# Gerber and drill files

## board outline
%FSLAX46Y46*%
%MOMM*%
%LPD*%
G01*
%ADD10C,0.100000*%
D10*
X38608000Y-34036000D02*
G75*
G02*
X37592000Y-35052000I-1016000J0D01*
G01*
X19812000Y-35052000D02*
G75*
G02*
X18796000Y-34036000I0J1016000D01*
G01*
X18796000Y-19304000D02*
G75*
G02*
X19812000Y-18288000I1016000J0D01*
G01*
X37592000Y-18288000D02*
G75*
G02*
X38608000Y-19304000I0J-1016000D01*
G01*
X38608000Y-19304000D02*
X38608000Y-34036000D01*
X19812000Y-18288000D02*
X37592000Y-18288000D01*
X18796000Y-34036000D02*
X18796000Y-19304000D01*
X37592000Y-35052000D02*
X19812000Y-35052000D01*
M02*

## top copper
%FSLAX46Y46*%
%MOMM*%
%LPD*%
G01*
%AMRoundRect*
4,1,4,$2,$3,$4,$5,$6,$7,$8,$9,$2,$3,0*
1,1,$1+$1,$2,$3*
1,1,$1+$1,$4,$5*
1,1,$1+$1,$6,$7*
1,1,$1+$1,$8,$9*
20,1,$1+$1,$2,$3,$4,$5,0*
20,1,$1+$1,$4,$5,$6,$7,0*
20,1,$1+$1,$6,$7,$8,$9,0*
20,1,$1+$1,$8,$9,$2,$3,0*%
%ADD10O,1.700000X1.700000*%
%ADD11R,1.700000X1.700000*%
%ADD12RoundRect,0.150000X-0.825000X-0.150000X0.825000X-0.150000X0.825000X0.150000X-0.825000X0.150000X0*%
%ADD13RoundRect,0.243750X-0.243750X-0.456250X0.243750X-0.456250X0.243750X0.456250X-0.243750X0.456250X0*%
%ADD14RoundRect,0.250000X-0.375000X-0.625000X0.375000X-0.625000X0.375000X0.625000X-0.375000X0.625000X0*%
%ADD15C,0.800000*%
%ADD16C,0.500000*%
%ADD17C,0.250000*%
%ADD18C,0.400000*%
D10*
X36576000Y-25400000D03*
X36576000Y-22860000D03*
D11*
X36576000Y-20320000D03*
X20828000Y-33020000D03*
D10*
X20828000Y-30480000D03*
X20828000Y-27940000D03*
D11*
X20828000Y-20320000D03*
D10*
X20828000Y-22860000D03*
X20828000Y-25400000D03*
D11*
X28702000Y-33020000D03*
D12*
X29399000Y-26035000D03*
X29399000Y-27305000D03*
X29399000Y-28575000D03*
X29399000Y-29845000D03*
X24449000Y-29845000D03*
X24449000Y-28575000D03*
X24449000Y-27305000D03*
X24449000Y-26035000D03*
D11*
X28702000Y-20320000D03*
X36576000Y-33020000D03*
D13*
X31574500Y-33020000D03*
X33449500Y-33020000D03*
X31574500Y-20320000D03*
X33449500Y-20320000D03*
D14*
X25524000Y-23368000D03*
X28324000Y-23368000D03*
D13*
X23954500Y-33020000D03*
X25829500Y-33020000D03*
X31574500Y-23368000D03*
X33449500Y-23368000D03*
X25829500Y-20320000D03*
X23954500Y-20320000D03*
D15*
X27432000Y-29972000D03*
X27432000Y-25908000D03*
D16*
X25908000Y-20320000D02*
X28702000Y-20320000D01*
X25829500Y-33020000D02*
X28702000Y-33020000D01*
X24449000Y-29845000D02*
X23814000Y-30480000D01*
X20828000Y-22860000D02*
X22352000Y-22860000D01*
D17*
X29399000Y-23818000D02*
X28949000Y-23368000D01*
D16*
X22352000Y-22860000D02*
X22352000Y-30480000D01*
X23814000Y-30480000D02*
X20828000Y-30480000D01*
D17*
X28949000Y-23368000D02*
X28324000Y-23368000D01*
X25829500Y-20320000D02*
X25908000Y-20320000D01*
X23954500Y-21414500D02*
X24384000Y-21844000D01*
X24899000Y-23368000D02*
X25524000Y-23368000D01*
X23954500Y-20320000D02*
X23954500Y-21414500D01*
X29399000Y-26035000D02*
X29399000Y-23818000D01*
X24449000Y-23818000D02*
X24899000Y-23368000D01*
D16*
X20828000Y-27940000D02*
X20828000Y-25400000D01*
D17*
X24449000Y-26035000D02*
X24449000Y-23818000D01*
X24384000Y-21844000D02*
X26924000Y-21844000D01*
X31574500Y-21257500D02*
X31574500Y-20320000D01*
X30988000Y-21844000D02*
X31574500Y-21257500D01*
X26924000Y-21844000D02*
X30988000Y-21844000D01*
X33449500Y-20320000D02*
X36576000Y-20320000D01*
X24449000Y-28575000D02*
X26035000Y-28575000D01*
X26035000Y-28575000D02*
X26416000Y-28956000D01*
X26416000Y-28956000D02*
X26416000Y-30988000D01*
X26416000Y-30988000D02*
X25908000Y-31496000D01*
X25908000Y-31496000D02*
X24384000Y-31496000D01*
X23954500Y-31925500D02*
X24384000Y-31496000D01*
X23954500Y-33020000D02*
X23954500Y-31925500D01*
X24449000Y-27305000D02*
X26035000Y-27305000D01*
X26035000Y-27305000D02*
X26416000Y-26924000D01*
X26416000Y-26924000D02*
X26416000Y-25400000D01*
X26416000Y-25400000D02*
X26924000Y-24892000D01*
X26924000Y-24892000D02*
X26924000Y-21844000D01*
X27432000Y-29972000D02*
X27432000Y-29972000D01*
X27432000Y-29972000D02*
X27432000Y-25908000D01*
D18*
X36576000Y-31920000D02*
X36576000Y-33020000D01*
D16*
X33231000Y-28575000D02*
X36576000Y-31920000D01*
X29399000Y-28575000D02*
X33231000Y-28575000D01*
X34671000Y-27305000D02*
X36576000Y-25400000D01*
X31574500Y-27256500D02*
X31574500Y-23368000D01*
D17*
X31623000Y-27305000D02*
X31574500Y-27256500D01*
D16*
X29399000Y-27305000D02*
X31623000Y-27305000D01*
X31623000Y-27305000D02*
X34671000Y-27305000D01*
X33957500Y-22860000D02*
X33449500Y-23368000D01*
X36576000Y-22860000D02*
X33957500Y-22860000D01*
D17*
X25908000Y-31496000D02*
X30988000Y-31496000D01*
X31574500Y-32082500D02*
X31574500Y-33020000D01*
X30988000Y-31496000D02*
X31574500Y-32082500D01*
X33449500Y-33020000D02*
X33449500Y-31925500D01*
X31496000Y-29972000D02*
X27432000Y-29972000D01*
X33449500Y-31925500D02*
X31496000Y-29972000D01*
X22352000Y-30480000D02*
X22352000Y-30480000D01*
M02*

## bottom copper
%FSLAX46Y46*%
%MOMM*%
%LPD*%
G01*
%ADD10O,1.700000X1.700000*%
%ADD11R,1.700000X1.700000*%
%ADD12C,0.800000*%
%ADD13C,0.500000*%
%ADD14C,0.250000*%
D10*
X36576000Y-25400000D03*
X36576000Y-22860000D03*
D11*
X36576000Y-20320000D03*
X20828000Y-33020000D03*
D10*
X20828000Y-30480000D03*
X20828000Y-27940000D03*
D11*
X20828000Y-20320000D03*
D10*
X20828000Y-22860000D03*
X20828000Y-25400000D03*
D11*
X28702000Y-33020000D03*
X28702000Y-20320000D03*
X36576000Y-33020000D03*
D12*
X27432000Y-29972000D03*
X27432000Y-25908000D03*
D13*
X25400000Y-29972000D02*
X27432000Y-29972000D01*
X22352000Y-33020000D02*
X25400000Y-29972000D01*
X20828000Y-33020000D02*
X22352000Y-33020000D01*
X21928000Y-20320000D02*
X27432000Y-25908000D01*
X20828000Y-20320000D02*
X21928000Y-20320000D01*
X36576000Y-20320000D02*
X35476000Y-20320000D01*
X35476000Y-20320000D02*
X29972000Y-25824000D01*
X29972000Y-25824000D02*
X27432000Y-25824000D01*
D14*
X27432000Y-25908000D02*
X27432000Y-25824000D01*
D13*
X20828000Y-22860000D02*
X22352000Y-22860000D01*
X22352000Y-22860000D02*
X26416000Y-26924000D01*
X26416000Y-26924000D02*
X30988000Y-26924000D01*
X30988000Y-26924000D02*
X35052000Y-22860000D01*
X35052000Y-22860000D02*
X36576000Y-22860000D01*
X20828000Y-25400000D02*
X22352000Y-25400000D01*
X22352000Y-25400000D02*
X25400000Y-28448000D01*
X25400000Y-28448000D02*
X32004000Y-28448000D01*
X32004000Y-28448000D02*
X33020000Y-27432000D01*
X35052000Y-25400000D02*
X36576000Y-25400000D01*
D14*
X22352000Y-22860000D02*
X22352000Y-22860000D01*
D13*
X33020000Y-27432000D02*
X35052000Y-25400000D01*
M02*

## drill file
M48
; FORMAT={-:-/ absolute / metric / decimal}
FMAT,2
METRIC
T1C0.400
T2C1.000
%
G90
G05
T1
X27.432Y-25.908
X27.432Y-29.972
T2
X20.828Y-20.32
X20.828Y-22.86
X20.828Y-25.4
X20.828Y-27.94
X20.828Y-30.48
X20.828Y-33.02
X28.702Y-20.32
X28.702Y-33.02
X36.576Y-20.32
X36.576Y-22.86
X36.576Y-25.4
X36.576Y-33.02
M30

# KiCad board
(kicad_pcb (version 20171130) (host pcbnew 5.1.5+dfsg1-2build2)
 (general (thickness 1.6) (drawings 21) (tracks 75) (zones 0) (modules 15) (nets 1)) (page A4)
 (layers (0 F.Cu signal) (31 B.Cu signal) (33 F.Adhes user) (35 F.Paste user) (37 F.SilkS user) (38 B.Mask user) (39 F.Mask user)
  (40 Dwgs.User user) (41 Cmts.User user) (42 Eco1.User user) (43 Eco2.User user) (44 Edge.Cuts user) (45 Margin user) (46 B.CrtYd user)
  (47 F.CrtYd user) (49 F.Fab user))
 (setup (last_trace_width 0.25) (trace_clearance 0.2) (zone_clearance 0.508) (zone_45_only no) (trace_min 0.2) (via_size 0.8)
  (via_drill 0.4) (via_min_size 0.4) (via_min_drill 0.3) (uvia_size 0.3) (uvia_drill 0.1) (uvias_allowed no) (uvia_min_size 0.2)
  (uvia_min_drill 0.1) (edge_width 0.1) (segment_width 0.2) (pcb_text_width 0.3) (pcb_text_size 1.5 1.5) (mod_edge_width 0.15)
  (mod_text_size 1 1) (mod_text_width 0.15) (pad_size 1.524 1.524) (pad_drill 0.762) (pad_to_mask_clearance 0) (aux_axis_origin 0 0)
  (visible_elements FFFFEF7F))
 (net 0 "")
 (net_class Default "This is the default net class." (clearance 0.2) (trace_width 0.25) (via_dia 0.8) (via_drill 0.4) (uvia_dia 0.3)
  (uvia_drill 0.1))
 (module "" (layer F.Cu) (at 26.67 28.448)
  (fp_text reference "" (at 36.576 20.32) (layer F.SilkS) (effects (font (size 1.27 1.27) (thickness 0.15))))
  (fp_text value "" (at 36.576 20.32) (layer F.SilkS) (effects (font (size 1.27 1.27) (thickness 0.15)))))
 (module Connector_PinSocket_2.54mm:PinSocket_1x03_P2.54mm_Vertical (layer F.Cu) (at 36.576 20.32)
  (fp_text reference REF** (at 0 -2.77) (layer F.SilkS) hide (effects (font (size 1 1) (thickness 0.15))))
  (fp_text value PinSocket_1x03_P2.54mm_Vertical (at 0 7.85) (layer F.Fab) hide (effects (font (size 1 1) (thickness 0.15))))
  (pad 3 thru_hole oval (at 0 5.08) (size 1.7 1.7) (drill 1) (layers *.Cu *.Mask))
  (pad 2 thru_hole oval (at 0 2.54) (size 1.7 1.7) (drill 1) (layers *.Cu *.Mask))
  (pad 1 thru_hole rect (at 0 0) (size 1.7 1.7) (drill 1) (layers *.Cu *.Mask)))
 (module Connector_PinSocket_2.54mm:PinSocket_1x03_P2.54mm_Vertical (layer F.Cu) (at 20.828 33.02 180)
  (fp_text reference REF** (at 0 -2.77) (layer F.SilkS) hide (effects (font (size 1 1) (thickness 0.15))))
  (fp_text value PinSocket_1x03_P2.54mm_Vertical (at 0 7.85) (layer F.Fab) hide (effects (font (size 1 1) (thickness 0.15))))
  (pad 1 thru_hole rect (at 0 0 180) (size 1.7 1.7) (drill 1) (layers *.Cu *.Mask))
  (pad 2 thru_hole oval (at 0 2.54 180) (size 1.7 1.7) (drill 1) (layers *.Cu *.Mask))
  (pad 3 thru_hole oval (at 0 5.08 180) (size 1.7 1.7) (drill 1) (layers *.Cu *.Mask)))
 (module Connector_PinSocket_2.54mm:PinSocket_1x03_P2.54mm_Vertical (layer F.Cu) (at 20.828 20.32)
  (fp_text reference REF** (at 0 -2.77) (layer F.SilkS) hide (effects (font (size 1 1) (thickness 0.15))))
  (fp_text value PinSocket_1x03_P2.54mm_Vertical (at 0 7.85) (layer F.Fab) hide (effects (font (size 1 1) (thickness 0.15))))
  (pad 1 thru_hole rect (at 0 0) (size 1.7 1.7) (drill 1) (layers *.Cu *.Mask))
  (pad 2 thru_hole oval (at 0 2.54) (size 1.7 1.7) (drill 1) (layers *.Cu *.Mask))
  (pad 3 thru_hole oval (at 0 5.08) (size 1.7 1.7) (drill 1) (layers *.Cu *.Mask)))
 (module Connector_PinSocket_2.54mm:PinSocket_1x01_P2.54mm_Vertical (layer F.Cu) (at 28.702 33.02)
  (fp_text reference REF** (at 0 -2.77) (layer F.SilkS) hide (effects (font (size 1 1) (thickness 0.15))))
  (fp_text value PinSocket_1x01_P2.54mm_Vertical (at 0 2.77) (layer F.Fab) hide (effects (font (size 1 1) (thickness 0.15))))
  (pad 1 thru_hole rect (at 0 0) (size 1.7 1.7) (drill 1) (layers *.Cu *.Mask)))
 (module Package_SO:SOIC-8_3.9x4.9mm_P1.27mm (layer F.Cu) (at 26.924 27.94)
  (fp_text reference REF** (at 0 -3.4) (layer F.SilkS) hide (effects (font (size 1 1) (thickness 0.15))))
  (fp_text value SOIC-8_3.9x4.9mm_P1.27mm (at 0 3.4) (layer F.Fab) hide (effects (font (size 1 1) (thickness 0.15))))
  (pad 8 smd roundrect (at 2.475 -1.905) (size 1.95 0.6) (layers F.Cu F.Paste F.Mask) (roundrect_rratio 0.25))
  (pad 7 smd roundrect (at 2.475 -0.635) (size 1.95 0.6) (layers F.Cu F.Paste F.Mask) (roundrect_rratio 0.25))
  (pad 6 smd roundrect (at 2.475 0.635) (size 1.95 0.6) (layers F.Cu F.Paste F.Mask) (roundrect_rratio 0.25))
  (pad 5 smd roundrect (at 2.475 1.905) (size 1.95 0.6) (layers F.Cu F.Paste F.Mask) (roundrect_rratio 0.25))
  (pad 4 smd roundrect (at -2.475 1.905) (size 1.95 0.6) (layers F.Cu F.Paste F.Mask) (roundrect_rratio 0.25))
  (pad 3 smd roundrect (at -2.475 0.635) (size 1.95 0.6) (layers F.Cu F.Paste F.Mask) (roundrect_rratio 0.25))
  (pad 2 smd roundrect (at -2.475 -0.635) (size 1.95 0.6) (layers F.Cu F.Paste F.Mask) (roundrect_rratio 0.25))
  (pad 1 smd roundrect (at -2.475 -1.905) (size 1.95 0.6) (layers F.Cu F.Paste F.Mask) (roundrect_rratio 0.25)))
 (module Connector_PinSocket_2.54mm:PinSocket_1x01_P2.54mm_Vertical (layer F.Cu) (at 28.702 20.32 180)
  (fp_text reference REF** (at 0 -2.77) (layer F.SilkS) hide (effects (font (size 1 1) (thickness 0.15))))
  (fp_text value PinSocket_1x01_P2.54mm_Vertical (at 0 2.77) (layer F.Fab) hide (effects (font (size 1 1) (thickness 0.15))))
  (pad 1 thru_hole rect (at 0 0 180) (size 1.7 1.7) (drill 1) (layers *.Cu *.Mask)))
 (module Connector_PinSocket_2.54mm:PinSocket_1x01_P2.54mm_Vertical (layer F.Cu) (at 36.576 33.02)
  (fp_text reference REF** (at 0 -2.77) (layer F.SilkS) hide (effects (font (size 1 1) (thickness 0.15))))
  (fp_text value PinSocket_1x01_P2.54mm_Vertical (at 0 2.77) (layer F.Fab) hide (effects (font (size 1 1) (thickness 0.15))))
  (pad 1 thru_hole rect (at 0 0) (size 1.7 1.7) (drill 1) (layers *.Cu *.Mask)))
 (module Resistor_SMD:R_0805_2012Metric (layer F.Cu) (at 32.512 33.02)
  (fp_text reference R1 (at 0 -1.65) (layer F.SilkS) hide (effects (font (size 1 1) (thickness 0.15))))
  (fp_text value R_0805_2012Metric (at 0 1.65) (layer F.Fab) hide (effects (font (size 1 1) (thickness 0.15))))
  (pad 1 smd roundrect (at -0.9375 0) (size 0.975 1.4) (layers F.Cu F.Paste F.Mask) (roundrect_rratio 0.25))
  (pad 2 smd roundrect (at 0.9375 0) (size 0.975 1.4) (layers F.Cu F.Paste F.Mask) (roundrect_rratio 0.25)))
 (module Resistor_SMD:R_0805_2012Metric (layer F.Cu) (at 32.512 20.32)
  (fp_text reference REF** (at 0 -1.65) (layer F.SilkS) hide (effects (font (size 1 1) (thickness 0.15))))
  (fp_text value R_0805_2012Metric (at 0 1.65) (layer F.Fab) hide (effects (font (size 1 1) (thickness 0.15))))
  (pad 1 smd roundrect (at -0.9375 0) (size 0.975 1.4) (layers F.Cu F.Paste F.Mask) (roundrect_rratio 0.25))
  (pad 2 smd roundrect (at 0.9375 0) (size 0.975 1.4) (layers F.Cu F.Paste F.Mask) (roundrect_rratio 0.25)))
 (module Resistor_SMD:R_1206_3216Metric (layer F.Cu) (at 26.924 23.368)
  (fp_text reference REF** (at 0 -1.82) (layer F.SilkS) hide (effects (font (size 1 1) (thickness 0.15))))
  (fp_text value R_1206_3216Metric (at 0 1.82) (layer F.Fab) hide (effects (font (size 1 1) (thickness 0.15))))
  (pad 1 smd roundrect (at -1.4 0) (size 1.25 1.75) (layers F.Cu F.Paste F.Mask) (roundrect_rratio 0.2))
  (pad 2 smd roundrect (at 1.4 0) (size 1.25 1.75) (layers F.Cu F.Paste F.Mask) (roundrect_rratio 0.2)))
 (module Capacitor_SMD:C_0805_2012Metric (layer F.Cu) (at 24.892 33.02)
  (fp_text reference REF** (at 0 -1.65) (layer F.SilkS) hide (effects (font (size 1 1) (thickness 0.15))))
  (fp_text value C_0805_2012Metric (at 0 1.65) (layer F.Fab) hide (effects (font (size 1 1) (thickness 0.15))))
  (pad 1 smd roundrect (at -0.9375 0) (size 0.975 1.4) (layers F.Cu F.Paste F.Mask) (roundrect_rratio 0.25))
  (pad 2 smd roundrect (at 0.9375 0) (size 0.975 1.4) (layers F.Cu F.Paste F.Mask) (roundrect_rratio 0.25)))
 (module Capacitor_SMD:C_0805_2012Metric (layer F.Cu) (at 32.512 23.368)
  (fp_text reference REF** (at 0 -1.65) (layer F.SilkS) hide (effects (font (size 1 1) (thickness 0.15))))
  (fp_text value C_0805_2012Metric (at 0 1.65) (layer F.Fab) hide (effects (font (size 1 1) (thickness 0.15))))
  (pad 1 smd roundrect (at -0.9375 0) (size 0.975 1.4) (layers F.Cu F.Paste F.Mask) (roundrect_rratio 0.25))
  (pad 2 smd roundrect (at 0.9375 0) (size 0.975 1.4) (layers F.Cu F.Paste F.Mask) (roundrect_rratio 0.25)))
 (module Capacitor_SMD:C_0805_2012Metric (layer F.Cu) (at 24.892 20.32)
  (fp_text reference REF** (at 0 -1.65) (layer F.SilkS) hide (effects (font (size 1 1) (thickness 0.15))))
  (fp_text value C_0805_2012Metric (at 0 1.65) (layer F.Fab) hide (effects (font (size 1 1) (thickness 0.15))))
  (pad 2 smd roundrect (at 0.9375 0) (size 0.975 1.4) (layers F.Cu F.Paste F.Mask) (roundrect_rratio 0.25))
  (pad 1 smd roundrect (at -0.9375 0) (size 0.975 1.4) (layers F.Cu F.Paste F.Mask) (roundrect_rratio 0.25)))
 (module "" (layer F.Cu) (at 33.02 36.83)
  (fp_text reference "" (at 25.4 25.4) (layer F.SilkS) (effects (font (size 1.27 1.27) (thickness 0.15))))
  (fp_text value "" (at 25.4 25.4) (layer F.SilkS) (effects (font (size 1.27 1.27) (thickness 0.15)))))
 (gr_arc (start 37.592 34.036) (end 37.592 35.052) (angle -90) (layer Edge.Cuts) (width 0.1))
 (gr_arc (start 19.812 34.036) (end 18.796 34.036) (angle -90) (layer Edge.Cuts) (width 0.1))
 (gr_arc (start 19.812 19.304) (end 19.812 18.288) (angle -90) (layer Edge.Cuts) (width 0.1))
 (gr_arc (start 37.592 19.304) (end 38.608 19.304) (angle -90) (layer Edge.Cuts) (width 0.1))
 (gr_line (start 38.608 19.304) (end 38.608 34.036) (layer Edge.Cuts) (width 0.1))
 (gr_line (start 19.812 18.288) (end 37.592 18.288) (layer Edge.Cuts) (width 0.1))
 (gr_line (start 18.796 34.036) (end 18.796 19.304) (layer Edge.Cuts) (width 0.1))
 (gr_line (start 37.592 35.052) (end 19.812 35.052) (layer Edge.Cuts) (width 0.1))
 (segment (start 25.908 20.32) (end 28.702 20.32) (width 0.5) (layer F.Cu) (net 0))
 (segment (start 25.8295 33.02) (end 28.702 33.02) (width 0.5) (layer F.Cu) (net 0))
 (segment (start 24.449 29.845) (end 23.814 30.48) (width 0.5) (layer F.Cu) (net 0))
 (segment (start 20.828 22.86) (end 22.352 22.86) (width 0.5) (layer F.Cu) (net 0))
 (segment (start 29.399 23.818) (end 28.949 23.368) (width 0.25) (layer F.Cu) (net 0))
 (segment (start 22.352 22.86) (end 22.352 30.48) (width 0.5) (layer F.Cu) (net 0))
 (segment (start 23.814 30.48) (end 20.828 30.48) (width 0.5) (layer F.Cu) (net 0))
 (segment (start 28.949 23.368) (end 28.324 23.368) (width 0.25) (layer F.Cu) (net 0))
 (segment (start 25.8295 20.32) (end 25.908 20.32) (width 0.25) (layer F.Cu) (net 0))
 (segment (start 23.9545 21.4145) (end 24.384 21.844) (width 0.25) (layer F.Cu) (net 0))
 (segment (start 24.899 23.368) (end 25.524 23.368) (width 0.25) (layer F.Cu) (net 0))
 (segment (start 23.9545 20.32) (end 23.9545 21.4145) (width 0.25) (layer F.Cu) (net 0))
 (segment (start 29.399 26.035) (end 29.399 23.818) (width 0.25) (layer F.Cu) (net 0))
 (segment (start 24.449 23.818) (end 24.899 23.368) (width 0.25) (layer F.Cu) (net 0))
 (segment (start 20.828 27.94) (end 20.828 25.4) (width 0.5) (layer F.Cu) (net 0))
 (segment (start 24.449 26.035) (end 24.449 23.818) (width 0.25) (layer F.Cu) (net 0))
 (segment (start 24.384 21.844) (end 26.924 21.844) (width 0.25) (layer F.Cu) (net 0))
 (segment (start 31.5745 21.2575) (end 31.5745 20.32) (width 0.25) (layer F.Cu) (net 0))
 (segment (start 30.988 21.844) (end 31.5745 21.2575) (width 0.25) (layer F.Cu) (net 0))
 (segment (start 26.924 21.844) (end 30.988 21.844) (width 0.25) (layer F.Cu) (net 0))
 (segment (start 33.4495 20.32) (end 36.576 20.32) (width 0.25) (layer F.Cu) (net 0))
 (segment (start 24.449 28.575) (end 26.035 28.575) (width 0.25) (layer F.Cu) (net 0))
 (segment (start 26.035 28.575) (end 26.416 28.956) (width 0.25) (layer F.Cu) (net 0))
 (segment (start 26.416 28.956) (end 26.416 30.988) (width 0.25) (layer F.Cu) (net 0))
 (segment (start 26.416 30.988) (end 25.908 31.496) (width 0.25) (layer F.Cu) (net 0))
 (segment (start 25.908 31.496) (end 24.384 31.496) (width 0.25) (layer F.Cu) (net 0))
 (segment (start 23.9545 31.9255) (end 24.384 31.496) (width 0.25) (layer F.Cu) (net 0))
 (segment (start 23.9545 33.02) (end 23.9545 31.9255) (width 0.25) (layer F.Cu) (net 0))
 (segment (start 24.449 27.305) (end 26.035 27.305) (width 0.25) (layer F.Cu) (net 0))
 (segment (start 26.035 27.305) (end 26.416 26.924) (width 0.25) (layer F.Cu) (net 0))
 (segment (start 26.416 26.924) (end 26.416 25.4) (width 0.25) (layer F.Cu) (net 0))
 (segment (start 26.416 25.4) (end 26.924 24.892) (width 0.25) (layer F.Cu) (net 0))
 (segment (start 26.924 24.892) (end 26.924 21.844) (width 0.25) (layer F.Cu) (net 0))
 (segment (start 27.432 29.972) (end 27.432 29.972) (width 0.25) (layer F.Cu) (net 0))
 (via (at 27.432 29.972) (size 0.8) (drill 0.4) (layers F.Cu B.Cu) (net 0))
 (segment (start 25.4 29.972) (end 27.432 29.972) (width 0.5) (layer B.Cu) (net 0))
 (segment (start 22.352 33.02) (end 25.4 29.972) (width 0.5) (layer B.Cu) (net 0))
 (segment (start 20.828 33.02) (end 22.352 33.02) (width 0.5) (layer B.Cu) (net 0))
 (segment (start 21.928 20.32) (end 27.432 25.908) (width 0.5) (layer B.Cu) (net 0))
 (segment (start 20.828 20.32) (end 21.928 20.32) (width 0.5) (layer B.Cu) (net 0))
 (segment (start 36.576 20.32) (end 35.476 20.32) (width 0.5) (layer B.Cu) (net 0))
 (segment (start 35.476 20.32) (end 29.972 25.824) (width 0.5) (layer B.Cu) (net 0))
 (segment (start 29.972 25.824) (end 27.432 25.824) (width 0.5) (layer B.Cu) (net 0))
 (segment (start 27.432 25.908) (end 27.432 25.824) (width 0.25) (layer B.Cu) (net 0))
 (via (at 27.432 25.908) (size 0.8) (drill 0.4) (layers F.Cu B.Cu) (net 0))
 (segment (start 27.432 29.972) (end 27.432 25.908) (width 0.25) (layer F.Cu) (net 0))
 (segment (start 36.576 31.92) (end 36.576 33.02) (width 0.4) (layer F.Cu) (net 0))
 (segment (start 33.231 28.575) (end 36.576 31.92) (width 0.5) (layer F.Cu) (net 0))
 (segment (start 29.399 28.575) (end 33.231 28.575) (width 0.5) (layer F.Cu) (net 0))
 (segment (start 20.828 22.86) (end 22.352 22.86) (width 0.5) (layer B.Cu) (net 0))
 (segment (start 22.352 22.86) (end 26.416 26.924) (width 0.5) (layer B.Cu) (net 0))
 (segment (start 26.416 26.924) (end 30.988 26.924) (width 0.5) (layer B.Cu) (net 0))
 (segment (start 30.988 26.924) (end 35.052 22.86) (width 0.5) (layer B.Cu) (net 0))
 (segment (start 35.052 22.86) (end 36.576 22.86) (width 0.5) (layer B.Cu) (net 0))
 (segment (start 20.828 25.4) (end 22.352 25.4) (width 0.5) (layer B.Cu) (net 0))
 (segment (start 22.352 25.4) (end 25.4 28.448) (width 0.5) (layer B.Cu) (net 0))
 (segment (start 25.4 28.448) (end 32.004 28.448) (width 0.5) (layer B.Cu) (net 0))
 (segment (start 32.004 28.448) (end 33.02 27.432) (width 0.5) (layer B.Cu) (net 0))
 (segment (start 35.052 25.4) (end 36.576 25.4) (width 0.5) (layer B.Cu) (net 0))
 (segment (start 34.671 27.305) (end 36.576 25.4) (width 0.5) (layer F.Cu) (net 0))
 (segment (start 31.5745 27.2565) (end 31.5745 23.368) (width 0.5) (layer F.Cu) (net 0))
 (segment (start 31.623 27.305) (end 31.5745 27.2565) (width 0.25) (layer F.Cu) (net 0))
 (segment (start 29.399 27.305) (end 31.623 27.305) (width 0.5) (layer F.Cu) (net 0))
 (segment (start 31.623 27.305) (end 34.671 27.305) (width 0.5) (layer F.Cu) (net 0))
 (segment (start 33.9575 22.86) (end 33.4495 23.368) (width 0.5) (layer F.Cu) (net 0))
 (segment (start 36.576 22.86) (end 33.9575 22.86) (width 0.5) (layer F.Cu) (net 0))
 (segment (start 25.908 31.496) (end 30.988 31.496) (width 0.25) (layer F.Cu) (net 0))
 (segment (start 31.5745 32.0825) (end 31.5745 33.02) (width 0.25) (layer F.Cu) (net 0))
 (segment (start 30.988 31.496) (end 31.5745 32.0825) (width 0.25) (layer F.Cu) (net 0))
 (segment (start 33.4495 33.02) (end 33.4495 31.9255) (width 0.25) (layer F.Cu) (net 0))
 (segment (start 31.496 29.972) (end 27.432 29.972) (width 0.25) (layer F.Cu) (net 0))
 (segment (start 33.4495 31.9255) (end 31.496 29.972) (width 0.25) (layer F.Cu) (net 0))
 (segment (start 22.352 22.86) (end 22.352 22.86) (width 0.25) (layer B.Cu) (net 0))
 (segment (start 33.02 27.432) (end 35.052 25.4) (width 0.5) (layer B.Cu) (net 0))
 (segment (start 22.352 30.48) (end 22.352 30.48) (width 0.25) (layer F.Cu) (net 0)))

